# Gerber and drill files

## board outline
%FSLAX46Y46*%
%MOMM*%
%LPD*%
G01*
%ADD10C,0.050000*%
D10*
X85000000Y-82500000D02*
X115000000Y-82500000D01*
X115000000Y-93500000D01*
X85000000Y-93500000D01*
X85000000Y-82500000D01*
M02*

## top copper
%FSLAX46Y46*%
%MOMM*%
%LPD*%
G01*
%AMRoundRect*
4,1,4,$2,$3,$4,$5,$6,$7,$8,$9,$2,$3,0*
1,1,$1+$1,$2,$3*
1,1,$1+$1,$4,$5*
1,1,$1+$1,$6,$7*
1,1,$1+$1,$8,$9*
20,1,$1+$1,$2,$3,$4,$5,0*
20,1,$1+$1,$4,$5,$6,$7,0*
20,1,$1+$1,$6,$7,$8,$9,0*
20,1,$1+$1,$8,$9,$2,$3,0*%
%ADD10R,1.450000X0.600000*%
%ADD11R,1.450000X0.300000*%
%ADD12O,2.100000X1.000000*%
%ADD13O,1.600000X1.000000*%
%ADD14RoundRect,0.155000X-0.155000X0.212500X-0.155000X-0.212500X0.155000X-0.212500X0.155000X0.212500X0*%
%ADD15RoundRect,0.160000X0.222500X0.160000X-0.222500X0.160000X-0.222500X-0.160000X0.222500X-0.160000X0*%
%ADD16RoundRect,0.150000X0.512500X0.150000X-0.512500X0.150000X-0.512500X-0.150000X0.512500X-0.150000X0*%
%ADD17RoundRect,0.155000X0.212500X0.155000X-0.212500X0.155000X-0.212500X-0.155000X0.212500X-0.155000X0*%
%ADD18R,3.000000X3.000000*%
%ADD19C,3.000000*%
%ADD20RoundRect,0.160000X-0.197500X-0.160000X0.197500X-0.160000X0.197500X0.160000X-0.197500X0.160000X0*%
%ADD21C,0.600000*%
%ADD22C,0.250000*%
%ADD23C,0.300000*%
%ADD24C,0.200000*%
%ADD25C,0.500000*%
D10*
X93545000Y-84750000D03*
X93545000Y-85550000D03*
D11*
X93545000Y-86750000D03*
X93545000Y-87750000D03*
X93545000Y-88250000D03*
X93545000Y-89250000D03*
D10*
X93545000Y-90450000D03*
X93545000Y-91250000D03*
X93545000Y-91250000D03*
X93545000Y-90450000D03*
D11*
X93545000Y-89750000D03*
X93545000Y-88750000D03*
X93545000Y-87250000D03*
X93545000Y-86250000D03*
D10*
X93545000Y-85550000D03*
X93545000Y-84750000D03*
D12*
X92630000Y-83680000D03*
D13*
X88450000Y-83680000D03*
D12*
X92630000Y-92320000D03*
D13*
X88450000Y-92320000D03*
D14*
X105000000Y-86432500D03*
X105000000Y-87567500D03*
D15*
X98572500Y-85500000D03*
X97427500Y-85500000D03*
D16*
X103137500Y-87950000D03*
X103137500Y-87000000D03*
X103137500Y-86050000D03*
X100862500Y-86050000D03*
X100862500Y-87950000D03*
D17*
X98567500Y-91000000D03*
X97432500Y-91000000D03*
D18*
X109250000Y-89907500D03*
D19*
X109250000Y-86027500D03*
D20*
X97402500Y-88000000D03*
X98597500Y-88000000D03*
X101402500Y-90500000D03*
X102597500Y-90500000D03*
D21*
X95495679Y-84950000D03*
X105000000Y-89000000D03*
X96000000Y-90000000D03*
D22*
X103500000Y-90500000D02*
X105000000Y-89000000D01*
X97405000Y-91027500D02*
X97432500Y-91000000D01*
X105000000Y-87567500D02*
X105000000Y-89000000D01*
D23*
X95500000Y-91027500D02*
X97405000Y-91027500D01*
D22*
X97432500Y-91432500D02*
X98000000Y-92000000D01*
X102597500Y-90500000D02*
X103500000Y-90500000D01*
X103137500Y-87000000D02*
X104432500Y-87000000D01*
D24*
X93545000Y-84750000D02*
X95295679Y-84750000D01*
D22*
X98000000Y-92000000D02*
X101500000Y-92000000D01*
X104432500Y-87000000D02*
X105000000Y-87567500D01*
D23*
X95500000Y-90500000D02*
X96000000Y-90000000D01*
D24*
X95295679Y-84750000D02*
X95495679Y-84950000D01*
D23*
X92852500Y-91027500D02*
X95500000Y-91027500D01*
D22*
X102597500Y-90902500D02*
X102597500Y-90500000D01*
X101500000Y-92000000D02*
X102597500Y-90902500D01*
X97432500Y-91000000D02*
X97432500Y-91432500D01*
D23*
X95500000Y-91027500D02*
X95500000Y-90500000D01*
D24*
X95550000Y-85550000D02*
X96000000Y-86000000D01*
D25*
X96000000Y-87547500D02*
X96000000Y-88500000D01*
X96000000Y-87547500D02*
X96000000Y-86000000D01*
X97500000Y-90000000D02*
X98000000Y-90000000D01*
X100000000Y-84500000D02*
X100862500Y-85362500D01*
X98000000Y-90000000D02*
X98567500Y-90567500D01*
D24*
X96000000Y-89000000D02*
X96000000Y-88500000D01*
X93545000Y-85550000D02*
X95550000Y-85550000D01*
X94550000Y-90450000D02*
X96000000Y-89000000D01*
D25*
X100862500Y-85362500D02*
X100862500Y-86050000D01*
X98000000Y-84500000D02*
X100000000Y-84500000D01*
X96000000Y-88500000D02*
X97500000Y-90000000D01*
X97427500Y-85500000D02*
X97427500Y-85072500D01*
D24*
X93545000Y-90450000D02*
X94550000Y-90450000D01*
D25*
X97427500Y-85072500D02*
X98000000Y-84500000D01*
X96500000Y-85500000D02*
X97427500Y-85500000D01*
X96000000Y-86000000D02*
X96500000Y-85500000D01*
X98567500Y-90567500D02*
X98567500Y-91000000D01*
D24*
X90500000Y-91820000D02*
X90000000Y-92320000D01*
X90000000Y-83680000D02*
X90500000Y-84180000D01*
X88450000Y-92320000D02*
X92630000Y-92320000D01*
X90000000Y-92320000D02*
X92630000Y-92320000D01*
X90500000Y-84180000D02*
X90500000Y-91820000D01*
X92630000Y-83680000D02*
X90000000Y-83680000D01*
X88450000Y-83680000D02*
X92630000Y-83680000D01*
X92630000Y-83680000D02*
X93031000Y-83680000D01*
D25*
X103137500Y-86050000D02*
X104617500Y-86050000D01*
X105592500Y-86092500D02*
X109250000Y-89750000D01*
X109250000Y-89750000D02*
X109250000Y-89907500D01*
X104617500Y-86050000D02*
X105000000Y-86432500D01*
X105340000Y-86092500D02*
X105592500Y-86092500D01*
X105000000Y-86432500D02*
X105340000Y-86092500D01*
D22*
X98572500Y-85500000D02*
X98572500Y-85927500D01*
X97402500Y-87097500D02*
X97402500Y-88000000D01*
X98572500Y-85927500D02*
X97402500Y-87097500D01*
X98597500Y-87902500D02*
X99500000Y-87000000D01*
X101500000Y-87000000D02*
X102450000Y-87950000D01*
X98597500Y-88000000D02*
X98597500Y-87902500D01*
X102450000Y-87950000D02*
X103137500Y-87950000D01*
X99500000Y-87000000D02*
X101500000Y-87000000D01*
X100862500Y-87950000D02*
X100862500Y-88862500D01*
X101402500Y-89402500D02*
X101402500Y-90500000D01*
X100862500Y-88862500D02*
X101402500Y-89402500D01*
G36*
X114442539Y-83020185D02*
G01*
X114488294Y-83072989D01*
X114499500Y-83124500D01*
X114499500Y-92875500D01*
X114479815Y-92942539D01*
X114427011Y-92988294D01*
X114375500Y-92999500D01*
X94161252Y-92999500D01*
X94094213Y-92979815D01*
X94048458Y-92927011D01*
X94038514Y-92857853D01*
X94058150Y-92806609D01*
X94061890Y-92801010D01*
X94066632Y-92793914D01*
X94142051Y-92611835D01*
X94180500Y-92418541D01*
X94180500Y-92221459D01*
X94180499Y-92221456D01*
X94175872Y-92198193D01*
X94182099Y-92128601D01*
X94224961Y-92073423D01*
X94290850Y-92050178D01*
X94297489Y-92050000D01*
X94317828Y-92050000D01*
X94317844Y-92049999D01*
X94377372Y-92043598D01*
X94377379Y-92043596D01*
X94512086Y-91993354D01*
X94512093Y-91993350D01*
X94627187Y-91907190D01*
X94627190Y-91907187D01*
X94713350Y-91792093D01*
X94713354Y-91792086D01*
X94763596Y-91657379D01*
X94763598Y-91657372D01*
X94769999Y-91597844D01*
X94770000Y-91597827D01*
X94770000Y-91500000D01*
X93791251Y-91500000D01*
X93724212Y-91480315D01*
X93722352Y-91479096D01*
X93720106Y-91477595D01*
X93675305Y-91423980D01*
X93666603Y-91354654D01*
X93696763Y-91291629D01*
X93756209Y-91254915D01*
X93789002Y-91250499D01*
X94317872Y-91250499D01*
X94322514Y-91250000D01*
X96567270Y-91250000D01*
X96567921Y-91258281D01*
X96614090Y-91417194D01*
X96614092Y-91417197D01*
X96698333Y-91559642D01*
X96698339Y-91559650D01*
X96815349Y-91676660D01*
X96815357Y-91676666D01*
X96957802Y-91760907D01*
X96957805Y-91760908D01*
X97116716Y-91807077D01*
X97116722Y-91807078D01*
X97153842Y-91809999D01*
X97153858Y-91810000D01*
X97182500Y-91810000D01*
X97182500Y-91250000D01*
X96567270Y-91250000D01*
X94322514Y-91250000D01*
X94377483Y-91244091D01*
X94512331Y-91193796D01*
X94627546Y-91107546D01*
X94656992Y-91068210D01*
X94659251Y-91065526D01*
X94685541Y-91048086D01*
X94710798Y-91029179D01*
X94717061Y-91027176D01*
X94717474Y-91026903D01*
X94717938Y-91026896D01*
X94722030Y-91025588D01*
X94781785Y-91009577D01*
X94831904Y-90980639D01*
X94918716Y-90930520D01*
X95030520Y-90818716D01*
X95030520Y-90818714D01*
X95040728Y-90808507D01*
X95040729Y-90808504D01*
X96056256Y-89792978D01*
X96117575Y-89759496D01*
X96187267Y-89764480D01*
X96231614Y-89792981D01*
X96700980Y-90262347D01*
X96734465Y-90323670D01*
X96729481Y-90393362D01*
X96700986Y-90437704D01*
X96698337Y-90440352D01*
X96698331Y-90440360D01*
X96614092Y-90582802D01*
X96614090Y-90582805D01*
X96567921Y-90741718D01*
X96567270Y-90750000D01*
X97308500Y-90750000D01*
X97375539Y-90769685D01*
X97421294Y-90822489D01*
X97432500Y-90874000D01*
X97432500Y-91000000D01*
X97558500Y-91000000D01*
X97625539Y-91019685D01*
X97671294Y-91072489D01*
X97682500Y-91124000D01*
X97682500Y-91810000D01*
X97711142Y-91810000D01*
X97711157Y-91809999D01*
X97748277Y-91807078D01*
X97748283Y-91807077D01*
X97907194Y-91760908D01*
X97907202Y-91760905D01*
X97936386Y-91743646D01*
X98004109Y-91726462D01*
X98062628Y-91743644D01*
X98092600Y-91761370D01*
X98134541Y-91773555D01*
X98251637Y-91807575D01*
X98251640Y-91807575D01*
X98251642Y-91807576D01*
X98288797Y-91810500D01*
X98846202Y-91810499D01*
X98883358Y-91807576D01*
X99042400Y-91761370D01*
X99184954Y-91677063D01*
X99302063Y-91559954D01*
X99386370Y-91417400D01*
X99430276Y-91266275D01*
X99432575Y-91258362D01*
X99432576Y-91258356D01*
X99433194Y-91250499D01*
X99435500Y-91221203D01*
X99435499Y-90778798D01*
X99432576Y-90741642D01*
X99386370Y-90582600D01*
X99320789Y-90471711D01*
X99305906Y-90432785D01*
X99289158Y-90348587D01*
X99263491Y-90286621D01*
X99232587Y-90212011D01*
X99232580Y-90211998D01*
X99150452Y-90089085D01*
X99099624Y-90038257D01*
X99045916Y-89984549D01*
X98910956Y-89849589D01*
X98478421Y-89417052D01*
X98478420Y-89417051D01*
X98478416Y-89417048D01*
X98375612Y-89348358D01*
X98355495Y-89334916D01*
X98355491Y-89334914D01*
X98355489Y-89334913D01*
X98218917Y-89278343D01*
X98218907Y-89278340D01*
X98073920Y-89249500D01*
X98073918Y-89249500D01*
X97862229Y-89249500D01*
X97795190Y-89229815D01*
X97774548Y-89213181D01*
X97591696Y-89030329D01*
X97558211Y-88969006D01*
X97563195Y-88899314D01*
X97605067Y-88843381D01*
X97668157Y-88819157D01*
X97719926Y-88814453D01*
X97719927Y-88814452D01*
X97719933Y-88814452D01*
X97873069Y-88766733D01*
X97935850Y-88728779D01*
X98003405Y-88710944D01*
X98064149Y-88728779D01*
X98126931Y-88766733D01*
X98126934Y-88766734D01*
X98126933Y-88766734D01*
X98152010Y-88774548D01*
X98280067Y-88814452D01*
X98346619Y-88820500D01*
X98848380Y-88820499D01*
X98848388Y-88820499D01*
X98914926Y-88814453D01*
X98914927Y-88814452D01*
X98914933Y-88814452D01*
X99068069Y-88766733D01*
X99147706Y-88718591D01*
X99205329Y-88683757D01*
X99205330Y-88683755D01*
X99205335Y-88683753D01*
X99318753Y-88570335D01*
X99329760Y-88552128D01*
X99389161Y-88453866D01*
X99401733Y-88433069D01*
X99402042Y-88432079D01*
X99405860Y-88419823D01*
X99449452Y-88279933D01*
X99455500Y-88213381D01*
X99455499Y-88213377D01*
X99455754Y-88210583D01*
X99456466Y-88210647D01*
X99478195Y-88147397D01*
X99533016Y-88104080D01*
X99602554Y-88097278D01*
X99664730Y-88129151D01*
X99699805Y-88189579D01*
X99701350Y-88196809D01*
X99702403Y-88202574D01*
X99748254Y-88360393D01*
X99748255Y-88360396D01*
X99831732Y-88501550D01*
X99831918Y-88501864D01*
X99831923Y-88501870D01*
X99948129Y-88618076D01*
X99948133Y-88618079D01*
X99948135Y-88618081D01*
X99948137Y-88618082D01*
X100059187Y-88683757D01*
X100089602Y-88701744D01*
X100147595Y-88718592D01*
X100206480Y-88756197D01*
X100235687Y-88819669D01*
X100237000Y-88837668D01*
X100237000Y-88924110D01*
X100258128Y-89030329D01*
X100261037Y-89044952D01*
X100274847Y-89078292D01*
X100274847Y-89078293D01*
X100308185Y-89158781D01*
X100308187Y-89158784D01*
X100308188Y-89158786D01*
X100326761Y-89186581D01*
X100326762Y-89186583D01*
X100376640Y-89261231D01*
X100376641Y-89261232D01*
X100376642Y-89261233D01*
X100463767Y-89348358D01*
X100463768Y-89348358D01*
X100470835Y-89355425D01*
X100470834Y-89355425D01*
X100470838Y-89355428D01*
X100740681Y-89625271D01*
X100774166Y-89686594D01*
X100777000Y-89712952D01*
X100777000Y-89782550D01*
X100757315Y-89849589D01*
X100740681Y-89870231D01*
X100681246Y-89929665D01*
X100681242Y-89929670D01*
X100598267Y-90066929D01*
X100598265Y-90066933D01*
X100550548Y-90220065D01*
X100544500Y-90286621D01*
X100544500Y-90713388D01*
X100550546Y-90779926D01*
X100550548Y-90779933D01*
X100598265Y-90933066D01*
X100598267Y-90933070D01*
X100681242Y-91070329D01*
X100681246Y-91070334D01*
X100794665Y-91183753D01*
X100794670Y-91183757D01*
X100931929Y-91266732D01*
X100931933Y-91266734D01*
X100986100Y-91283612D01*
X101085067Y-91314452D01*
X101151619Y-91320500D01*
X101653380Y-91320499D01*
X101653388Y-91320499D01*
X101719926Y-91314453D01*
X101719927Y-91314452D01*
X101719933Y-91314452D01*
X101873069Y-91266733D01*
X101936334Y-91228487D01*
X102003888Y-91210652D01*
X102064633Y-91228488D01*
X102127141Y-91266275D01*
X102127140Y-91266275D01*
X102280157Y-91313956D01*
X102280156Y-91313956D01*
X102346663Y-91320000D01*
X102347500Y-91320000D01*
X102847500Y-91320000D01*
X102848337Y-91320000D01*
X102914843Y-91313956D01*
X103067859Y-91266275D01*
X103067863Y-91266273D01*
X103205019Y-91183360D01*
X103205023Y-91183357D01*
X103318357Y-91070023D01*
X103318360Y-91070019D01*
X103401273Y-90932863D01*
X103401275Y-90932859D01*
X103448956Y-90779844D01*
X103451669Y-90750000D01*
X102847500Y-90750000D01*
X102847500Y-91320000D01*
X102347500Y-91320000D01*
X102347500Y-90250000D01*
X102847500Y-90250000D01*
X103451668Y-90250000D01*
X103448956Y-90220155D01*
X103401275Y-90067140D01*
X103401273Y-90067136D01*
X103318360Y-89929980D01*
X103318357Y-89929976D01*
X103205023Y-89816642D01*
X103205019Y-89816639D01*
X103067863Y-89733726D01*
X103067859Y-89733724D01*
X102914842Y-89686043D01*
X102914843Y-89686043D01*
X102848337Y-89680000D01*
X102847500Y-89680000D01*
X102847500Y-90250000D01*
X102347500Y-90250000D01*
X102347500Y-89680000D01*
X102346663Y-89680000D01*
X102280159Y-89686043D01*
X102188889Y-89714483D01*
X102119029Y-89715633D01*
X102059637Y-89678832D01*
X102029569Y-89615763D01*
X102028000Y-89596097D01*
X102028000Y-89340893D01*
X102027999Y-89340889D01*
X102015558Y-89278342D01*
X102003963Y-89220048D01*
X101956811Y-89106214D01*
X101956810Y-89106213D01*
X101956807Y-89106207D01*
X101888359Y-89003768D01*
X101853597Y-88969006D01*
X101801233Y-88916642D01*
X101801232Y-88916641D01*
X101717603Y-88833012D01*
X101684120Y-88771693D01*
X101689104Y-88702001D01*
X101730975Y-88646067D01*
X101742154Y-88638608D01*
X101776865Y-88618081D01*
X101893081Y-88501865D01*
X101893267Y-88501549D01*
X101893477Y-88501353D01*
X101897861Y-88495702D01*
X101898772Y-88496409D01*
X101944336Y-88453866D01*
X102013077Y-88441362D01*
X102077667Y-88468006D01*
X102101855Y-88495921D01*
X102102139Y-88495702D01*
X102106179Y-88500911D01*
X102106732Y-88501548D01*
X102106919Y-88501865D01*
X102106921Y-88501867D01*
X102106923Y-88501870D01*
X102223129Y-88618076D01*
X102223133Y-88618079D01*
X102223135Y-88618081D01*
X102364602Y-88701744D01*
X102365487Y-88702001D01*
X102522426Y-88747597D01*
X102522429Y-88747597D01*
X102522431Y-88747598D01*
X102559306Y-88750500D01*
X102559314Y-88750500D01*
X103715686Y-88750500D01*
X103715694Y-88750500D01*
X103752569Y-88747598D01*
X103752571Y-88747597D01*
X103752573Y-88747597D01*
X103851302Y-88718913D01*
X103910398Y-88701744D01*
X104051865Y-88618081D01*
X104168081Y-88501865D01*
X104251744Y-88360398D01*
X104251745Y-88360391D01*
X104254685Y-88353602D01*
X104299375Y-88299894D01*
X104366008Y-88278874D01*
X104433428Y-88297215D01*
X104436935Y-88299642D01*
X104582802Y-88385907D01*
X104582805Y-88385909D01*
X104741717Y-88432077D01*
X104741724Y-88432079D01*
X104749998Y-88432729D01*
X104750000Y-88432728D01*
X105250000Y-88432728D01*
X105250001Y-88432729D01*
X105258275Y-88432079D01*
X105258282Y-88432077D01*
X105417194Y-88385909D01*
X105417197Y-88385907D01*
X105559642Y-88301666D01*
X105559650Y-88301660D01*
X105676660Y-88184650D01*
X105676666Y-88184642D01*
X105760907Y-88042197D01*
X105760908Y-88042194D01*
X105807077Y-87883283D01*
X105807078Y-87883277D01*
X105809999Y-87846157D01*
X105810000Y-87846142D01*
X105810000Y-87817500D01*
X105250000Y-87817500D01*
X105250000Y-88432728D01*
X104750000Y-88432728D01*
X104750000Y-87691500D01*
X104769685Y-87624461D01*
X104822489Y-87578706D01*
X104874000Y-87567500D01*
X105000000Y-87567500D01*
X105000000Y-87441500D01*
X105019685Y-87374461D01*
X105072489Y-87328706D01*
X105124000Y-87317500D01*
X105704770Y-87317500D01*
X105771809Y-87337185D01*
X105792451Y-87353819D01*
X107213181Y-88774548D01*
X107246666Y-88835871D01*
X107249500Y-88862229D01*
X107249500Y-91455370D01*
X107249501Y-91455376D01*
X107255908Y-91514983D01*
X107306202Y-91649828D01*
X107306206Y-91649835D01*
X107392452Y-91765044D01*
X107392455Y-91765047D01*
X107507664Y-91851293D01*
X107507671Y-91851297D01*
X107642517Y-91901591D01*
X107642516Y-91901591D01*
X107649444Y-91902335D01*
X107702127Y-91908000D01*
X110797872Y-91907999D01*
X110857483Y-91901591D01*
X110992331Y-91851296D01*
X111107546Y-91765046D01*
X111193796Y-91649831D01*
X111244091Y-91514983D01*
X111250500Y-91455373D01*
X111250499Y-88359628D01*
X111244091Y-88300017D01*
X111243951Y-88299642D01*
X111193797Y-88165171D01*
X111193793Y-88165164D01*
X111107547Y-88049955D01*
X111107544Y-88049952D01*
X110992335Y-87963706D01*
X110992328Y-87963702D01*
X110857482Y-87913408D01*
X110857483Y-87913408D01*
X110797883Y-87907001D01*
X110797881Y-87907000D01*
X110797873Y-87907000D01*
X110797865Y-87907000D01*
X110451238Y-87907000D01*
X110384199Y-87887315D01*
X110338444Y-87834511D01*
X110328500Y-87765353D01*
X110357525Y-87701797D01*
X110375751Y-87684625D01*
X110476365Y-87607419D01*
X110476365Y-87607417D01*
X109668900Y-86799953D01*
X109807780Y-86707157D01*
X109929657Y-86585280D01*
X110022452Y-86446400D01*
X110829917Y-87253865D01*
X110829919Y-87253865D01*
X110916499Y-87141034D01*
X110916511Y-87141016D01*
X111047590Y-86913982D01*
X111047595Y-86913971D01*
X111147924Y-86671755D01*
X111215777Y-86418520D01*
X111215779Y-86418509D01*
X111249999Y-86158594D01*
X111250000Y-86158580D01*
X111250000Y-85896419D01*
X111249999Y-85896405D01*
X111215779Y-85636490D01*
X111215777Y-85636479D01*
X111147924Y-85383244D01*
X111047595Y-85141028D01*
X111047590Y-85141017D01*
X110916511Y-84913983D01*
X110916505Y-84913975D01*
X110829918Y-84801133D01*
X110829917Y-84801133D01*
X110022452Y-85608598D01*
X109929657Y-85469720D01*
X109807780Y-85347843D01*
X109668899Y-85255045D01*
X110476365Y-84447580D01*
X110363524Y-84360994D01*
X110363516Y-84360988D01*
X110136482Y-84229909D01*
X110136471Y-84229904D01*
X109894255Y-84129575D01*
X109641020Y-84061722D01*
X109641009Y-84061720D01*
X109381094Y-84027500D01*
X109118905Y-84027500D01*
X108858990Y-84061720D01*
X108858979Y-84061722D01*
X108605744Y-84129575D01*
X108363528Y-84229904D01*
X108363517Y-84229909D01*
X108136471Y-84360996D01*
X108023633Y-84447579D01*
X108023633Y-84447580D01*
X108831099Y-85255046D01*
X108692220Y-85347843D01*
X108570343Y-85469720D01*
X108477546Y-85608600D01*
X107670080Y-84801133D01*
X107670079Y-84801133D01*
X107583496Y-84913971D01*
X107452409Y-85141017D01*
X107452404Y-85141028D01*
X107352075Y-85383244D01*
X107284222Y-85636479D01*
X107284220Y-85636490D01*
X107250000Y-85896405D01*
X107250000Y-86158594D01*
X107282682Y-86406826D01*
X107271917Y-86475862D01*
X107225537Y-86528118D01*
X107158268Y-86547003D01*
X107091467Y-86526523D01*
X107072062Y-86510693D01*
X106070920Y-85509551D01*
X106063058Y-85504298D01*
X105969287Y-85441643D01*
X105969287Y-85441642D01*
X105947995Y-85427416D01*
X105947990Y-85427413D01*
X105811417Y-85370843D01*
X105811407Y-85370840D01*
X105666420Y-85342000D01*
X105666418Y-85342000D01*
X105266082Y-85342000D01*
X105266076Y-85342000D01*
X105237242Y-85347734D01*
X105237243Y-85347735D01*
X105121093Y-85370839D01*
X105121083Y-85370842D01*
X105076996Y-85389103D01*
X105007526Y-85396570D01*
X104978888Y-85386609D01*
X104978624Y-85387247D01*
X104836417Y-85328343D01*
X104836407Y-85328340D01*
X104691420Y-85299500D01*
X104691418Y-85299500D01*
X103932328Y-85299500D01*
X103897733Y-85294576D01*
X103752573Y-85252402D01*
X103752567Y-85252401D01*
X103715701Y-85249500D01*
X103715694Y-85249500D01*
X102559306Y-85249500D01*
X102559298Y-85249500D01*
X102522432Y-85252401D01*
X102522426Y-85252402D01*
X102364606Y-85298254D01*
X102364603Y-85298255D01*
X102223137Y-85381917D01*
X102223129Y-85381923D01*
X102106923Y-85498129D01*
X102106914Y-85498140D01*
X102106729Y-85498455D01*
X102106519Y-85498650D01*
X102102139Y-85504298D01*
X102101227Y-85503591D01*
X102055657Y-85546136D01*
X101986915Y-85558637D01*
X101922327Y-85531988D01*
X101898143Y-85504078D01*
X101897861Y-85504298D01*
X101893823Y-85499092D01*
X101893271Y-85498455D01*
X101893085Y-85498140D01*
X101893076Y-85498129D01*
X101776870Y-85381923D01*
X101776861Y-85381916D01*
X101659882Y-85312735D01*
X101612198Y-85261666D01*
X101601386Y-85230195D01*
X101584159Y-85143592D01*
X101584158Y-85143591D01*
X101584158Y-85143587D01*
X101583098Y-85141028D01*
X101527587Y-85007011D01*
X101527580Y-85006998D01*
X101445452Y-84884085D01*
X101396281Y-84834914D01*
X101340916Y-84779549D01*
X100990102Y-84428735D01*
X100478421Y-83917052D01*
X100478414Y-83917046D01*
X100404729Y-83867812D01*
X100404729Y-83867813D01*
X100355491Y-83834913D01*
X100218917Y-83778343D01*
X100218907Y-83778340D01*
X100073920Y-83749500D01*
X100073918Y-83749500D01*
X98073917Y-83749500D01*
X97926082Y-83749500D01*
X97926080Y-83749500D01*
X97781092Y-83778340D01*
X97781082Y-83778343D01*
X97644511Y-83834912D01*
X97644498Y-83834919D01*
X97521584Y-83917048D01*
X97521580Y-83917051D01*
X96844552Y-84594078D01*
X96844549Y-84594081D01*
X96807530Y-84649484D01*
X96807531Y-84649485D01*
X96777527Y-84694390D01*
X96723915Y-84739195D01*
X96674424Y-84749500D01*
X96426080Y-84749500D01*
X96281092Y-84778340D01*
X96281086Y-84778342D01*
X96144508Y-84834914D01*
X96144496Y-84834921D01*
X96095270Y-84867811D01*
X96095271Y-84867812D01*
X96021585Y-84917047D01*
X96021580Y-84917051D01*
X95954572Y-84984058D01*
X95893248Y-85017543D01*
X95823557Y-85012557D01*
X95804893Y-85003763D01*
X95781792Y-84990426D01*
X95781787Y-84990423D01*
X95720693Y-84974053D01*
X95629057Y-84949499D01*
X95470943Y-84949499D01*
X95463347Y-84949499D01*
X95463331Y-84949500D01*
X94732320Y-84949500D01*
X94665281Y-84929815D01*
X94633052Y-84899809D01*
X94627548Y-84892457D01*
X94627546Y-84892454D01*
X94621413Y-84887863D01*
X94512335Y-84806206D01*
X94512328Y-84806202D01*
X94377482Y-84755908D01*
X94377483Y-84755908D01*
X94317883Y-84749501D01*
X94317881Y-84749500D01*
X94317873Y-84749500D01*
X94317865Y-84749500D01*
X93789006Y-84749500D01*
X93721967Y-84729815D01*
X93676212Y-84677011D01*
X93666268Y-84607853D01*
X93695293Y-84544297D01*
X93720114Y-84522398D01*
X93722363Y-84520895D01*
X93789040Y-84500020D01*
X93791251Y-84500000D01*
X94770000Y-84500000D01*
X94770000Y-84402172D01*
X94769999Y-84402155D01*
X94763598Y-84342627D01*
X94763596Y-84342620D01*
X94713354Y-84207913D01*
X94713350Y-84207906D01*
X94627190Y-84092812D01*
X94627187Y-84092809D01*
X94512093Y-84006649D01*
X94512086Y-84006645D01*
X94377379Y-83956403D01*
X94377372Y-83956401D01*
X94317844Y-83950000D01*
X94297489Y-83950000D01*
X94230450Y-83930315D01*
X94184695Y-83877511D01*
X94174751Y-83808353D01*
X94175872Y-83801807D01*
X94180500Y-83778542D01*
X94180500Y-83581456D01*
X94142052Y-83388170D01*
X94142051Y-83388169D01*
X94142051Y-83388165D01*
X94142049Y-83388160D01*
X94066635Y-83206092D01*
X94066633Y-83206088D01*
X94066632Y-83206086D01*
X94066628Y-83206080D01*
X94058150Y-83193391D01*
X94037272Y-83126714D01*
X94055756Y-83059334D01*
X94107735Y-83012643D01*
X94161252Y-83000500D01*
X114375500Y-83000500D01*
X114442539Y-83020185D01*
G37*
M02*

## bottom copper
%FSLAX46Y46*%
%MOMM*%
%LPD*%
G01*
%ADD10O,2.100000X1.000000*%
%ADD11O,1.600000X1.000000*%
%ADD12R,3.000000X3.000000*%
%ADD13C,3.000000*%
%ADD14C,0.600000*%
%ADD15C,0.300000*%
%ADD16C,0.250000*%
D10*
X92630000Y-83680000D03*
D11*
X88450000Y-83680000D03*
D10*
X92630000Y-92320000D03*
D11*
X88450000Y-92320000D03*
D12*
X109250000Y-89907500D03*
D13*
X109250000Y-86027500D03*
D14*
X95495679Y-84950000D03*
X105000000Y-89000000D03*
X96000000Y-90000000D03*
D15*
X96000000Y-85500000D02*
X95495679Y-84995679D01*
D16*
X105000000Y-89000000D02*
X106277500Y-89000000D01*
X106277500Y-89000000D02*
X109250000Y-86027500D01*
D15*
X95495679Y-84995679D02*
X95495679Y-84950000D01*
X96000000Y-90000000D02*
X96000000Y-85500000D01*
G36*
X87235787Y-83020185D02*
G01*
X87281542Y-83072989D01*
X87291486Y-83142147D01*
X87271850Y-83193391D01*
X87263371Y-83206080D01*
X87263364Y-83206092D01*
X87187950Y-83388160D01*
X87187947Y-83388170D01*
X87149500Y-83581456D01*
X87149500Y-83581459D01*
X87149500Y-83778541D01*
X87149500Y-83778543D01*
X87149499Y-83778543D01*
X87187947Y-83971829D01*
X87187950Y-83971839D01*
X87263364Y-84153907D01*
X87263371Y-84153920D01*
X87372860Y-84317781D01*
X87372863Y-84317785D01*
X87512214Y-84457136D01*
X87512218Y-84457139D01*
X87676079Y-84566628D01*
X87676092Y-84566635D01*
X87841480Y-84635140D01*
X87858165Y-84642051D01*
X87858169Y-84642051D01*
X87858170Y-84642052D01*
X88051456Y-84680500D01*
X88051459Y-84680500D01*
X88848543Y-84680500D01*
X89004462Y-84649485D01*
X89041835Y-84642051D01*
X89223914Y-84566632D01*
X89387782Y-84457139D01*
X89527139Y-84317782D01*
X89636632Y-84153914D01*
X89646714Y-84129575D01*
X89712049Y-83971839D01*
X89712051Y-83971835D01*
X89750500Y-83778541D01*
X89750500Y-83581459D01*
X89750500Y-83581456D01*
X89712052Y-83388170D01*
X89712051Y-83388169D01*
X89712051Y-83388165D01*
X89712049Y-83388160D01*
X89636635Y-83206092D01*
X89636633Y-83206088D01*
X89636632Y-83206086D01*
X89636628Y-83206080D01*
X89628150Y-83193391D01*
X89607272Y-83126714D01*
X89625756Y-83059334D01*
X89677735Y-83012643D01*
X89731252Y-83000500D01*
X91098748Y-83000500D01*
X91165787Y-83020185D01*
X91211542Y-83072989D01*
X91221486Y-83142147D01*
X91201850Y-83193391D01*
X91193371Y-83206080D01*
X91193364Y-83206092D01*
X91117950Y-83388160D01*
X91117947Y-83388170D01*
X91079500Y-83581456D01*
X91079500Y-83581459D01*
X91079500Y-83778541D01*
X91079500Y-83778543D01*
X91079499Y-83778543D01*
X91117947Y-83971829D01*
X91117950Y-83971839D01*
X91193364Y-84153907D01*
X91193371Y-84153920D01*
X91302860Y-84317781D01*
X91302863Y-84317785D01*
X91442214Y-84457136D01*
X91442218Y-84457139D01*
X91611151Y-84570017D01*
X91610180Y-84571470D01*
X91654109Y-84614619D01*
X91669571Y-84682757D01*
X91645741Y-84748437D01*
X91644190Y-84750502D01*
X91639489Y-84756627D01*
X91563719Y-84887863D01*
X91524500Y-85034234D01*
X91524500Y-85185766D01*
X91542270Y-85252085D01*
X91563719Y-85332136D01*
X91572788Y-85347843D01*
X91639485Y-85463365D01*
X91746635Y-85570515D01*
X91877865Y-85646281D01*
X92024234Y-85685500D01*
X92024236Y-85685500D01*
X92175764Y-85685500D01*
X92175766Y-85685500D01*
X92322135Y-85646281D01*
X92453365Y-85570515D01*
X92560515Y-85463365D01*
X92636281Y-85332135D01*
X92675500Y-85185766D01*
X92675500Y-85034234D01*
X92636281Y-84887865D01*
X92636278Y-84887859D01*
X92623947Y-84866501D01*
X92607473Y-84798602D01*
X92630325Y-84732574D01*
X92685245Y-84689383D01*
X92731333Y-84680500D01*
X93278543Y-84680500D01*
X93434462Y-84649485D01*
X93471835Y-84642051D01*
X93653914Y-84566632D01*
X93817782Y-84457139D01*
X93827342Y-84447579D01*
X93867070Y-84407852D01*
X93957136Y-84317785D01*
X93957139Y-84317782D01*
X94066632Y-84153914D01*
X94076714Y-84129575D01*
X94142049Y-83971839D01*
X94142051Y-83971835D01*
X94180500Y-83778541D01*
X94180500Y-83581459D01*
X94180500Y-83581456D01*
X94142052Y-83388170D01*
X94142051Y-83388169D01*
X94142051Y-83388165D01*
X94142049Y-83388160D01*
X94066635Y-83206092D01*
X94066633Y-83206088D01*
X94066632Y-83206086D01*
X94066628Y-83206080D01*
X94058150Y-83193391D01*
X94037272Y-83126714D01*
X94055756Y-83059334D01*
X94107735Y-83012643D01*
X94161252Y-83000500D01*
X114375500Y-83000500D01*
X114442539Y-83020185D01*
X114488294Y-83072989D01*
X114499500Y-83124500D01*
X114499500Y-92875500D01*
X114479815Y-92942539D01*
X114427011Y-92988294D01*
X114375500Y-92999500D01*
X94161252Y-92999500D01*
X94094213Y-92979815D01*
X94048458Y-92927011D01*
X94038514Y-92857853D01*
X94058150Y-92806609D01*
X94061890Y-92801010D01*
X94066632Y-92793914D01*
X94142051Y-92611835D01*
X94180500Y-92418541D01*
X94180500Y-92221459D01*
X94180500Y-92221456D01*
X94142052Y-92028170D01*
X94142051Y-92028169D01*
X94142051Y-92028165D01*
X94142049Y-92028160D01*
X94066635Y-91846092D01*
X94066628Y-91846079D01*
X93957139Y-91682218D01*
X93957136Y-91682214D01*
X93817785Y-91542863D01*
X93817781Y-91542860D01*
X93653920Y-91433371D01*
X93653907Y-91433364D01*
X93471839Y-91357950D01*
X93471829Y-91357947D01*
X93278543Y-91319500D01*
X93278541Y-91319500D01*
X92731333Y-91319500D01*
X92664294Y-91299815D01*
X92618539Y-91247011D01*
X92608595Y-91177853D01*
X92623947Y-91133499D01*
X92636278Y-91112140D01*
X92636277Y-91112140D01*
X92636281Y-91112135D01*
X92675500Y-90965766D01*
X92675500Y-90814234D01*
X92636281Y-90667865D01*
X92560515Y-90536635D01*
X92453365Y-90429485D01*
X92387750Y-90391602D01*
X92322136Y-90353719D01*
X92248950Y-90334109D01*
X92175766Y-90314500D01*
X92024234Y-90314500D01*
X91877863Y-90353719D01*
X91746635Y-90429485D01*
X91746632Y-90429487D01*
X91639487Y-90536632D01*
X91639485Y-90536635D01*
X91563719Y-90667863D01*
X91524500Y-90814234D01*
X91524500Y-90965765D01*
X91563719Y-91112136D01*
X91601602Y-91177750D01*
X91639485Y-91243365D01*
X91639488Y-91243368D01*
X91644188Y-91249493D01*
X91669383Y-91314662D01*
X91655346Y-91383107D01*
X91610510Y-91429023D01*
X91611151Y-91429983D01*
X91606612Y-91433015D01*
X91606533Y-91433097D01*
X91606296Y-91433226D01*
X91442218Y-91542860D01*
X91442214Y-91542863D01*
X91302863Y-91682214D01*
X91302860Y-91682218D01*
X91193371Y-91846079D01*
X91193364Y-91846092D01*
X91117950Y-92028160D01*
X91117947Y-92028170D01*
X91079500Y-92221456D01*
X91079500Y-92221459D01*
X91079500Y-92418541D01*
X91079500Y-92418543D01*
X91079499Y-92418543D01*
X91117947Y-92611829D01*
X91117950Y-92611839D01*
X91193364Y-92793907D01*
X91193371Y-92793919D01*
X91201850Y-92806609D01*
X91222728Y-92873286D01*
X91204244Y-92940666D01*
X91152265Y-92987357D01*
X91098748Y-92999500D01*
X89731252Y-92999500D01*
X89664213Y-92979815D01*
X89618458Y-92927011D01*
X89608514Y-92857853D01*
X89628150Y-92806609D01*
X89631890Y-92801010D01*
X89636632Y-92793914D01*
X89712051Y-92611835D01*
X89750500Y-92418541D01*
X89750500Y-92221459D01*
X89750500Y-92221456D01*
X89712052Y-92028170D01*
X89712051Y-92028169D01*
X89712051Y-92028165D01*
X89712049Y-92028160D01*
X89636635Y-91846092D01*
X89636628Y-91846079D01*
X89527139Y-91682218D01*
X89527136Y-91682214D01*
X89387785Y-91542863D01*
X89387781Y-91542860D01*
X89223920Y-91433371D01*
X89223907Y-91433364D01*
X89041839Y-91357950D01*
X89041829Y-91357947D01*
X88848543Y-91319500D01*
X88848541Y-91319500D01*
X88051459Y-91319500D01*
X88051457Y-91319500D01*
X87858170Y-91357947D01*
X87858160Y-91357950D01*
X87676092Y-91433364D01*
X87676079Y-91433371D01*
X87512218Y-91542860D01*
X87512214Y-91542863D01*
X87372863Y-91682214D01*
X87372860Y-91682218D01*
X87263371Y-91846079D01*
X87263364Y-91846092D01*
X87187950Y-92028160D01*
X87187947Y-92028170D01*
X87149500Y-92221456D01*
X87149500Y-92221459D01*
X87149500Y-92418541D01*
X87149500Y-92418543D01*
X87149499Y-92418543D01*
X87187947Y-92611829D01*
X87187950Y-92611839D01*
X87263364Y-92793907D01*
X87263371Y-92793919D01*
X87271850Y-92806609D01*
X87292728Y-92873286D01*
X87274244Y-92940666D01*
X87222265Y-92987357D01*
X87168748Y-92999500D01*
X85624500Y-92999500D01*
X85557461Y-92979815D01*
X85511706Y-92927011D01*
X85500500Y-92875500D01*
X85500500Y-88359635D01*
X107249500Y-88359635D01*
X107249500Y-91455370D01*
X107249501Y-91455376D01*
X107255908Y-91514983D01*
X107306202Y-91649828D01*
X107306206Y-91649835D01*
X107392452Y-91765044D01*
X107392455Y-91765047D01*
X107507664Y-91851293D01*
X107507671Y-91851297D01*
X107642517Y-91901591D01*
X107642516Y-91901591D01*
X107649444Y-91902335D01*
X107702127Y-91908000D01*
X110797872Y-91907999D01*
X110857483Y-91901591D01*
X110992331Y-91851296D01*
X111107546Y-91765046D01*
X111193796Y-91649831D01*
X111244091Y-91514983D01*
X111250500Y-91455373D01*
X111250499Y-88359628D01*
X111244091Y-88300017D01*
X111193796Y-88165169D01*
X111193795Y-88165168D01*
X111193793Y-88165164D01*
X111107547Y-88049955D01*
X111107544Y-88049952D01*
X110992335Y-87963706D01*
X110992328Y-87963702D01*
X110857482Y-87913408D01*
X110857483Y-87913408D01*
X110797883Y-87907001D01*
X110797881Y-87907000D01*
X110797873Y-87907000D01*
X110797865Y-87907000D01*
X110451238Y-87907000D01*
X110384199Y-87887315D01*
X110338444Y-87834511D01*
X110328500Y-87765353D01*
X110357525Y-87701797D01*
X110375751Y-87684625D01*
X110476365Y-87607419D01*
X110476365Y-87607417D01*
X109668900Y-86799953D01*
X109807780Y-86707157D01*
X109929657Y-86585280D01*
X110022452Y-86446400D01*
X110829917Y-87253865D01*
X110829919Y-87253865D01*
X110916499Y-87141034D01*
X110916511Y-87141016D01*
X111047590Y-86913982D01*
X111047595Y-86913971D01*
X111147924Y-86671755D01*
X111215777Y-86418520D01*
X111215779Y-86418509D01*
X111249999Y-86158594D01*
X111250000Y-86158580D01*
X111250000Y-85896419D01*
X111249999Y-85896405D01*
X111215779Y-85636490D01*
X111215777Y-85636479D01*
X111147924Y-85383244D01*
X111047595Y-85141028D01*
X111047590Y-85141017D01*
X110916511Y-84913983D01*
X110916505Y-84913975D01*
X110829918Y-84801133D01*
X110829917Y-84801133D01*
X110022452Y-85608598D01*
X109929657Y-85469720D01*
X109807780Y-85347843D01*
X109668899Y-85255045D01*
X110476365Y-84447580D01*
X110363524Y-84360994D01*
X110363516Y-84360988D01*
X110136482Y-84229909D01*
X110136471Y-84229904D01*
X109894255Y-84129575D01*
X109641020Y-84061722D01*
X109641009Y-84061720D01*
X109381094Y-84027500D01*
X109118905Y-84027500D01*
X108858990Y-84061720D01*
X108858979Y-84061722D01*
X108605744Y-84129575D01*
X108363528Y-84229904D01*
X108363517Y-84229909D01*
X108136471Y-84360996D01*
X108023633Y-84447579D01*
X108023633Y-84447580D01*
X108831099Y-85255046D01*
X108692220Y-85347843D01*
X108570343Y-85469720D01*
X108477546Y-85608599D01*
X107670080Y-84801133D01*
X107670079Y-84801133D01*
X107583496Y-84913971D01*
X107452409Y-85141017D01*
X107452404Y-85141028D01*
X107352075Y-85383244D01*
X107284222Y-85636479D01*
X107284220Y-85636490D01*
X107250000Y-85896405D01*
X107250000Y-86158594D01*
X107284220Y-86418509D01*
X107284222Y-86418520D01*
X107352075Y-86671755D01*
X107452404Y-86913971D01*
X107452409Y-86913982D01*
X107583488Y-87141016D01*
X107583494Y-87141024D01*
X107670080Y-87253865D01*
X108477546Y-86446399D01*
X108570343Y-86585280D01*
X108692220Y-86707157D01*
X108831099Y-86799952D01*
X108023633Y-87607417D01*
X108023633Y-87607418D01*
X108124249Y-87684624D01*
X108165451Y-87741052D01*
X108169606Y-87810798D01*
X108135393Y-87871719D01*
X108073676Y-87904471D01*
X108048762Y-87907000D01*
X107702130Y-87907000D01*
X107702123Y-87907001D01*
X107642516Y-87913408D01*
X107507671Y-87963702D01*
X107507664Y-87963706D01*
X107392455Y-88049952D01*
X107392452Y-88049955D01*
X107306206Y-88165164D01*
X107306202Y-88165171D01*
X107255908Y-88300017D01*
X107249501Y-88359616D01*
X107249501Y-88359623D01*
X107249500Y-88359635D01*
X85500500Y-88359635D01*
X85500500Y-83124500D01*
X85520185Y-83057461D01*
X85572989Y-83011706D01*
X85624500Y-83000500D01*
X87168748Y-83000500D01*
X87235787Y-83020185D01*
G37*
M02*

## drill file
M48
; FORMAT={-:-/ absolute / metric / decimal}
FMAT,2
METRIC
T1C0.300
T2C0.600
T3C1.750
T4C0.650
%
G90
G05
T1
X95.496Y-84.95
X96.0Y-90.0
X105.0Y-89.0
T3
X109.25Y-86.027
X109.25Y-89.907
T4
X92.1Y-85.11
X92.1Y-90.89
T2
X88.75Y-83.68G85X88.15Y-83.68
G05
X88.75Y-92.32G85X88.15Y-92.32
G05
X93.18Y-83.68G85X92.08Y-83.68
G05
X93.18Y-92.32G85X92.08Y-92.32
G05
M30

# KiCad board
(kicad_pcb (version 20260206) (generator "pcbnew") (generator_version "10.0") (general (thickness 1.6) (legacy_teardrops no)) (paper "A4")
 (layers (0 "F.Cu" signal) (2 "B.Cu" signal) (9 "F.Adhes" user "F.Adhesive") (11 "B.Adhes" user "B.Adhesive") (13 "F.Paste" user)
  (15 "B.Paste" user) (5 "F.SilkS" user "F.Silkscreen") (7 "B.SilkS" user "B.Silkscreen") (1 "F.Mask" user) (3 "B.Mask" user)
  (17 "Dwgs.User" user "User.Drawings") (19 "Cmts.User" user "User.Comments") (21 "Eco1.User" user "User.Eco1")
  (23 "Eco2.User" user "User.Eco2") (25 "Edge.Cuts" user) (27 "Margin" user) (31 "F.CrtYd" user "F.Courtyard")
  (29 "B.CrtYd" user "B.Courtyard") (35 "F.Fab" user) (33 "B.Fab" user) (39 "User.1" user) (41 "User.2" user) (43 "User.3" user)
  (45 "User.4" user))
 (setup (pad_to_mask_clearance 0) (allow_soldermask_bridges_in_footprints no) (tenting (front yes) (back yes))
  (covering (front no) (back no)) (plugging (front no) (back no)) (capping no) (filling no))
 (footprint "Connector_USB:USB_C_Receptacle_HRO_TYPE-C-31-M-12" (layer "F.Cu") (at 89.5 88 -90)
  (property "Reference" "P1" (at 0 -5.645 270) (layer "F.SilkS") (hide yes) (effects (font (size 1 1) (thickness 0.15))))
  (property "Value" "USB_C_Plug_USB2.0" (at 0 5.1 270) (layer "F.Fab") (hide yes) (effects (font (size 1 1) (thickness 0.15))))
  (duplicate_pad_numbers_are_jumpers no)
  (pad "" np_thru_hole circle (at -2.89 -2.6 270) (size 0.65 0.65) (drill 0.65) (layers "*.Cu" "*.Mask"))
  (pad "" np_thru_hole circle (at 2.89 -2.6 270) (size 0.65 0.65) (drill 0.65) (layers "*.Cu" "*.Mask"))
  (pad "A1" smd rect (at -3.25 -4.045 270) (size 0.6 1.45) (layers "F.Cu" "F.Mask" "F.Paste") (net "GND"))
  (pad "A4" smd rect (at -2.45 -4.045 270) (size 0.6 1.45) (layers "F.Cu" "F.Mask" "F.Paste") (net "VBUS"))
  (pad "A5" smd rect (at -1.25 -4.045 270) (size 0.3 1.45) (layers "F.Cu" "F.Mask" "F.Paste") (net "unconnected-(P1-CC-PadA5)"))
  (pad "A6" smd rect (at -0.25 -4.045 270) (size 0.3 1.45) (layers "F.Cu" "F.Mask" "F.Paste") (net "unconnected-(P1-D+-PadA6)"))
  (pad "A7" smd rect (at 0.25 -4.045 270) (size 0.3 1.45) (layers "F.Cu" "F.Mask" "F.Paste") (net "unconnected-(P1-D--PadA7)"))
  (pad "A8" smd rect (at 1.25 -4.045 270) (size 0.3 1.45) (layers "F.Cu" "F.Mask" "F.Paste"))
  (pad "A9" smd rect (at 2.45 -4.045 270) (size 0.6 1.45) (layers "F.Cu" "F.Mask" "F.Paste") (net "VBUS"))
  (pad "A12" smd rect (at 3.25 -4.045 270) (size 0.6 1.45) (layers "F.Cu" "F.Mask" "F.Paste") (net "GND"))
  (pad "B1" smd rect (at 3.25 -4.045 270) (size 0.6 1.45) (layers "F.Cu" "F.Mask" "F.Paste") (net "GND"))
  (pad "B4" smd rect (at 2.45 -4.045 270) (size 0.6 1.45) (layers "F.Cu" "F.Mask" "F.Paste") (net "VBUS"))
  (pad "B5" smd rect (at 1.75 -4.045 270) (size 0.3 1.45) (layers "F.Cu" "F.Mask" "F.Paste") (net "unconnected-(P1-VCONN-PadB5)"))
  (pad "B6" smd rect (at 0.75 -4.045 270) (size 0.3 1.45) (layers "F.Cu" "F.Mask" "F.Paste"))
  (pad "B7" smd rect (at -0.75 -4.045 270) (size 0.3 1.45) (layers "F.Cu" "F.Mask" "F.Paste"))
  (pad "B8" smd rect (at -1.75 -4.045 270) (size 0.3 1.45) (layers "F.Cu" "F.Mask" "F.Paste"))
  (pad "B9" smd rect (at -2.45 -4.045 270) (size 0.6 1.45) (layers "F.Cu" "F.Mask" "F.Paste") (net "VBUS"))
  (pad "B12" smd rect (at -3.25 -4.045 270) (size 0.6 1.45) (layers "F.Cu" "F.Mask" "F.Paste") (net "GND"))
  (pad "S1" thru_hole oval (at -4.32 -3.13 270) (size 1 2.1) (drill oval 0.6 1.7) (layers "*.Cu" "*.Mask") (remove_unused_layers no)
   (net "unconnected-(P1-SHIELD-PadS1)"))
  (pad "S1" thru_hole oval (at -4.32 1.05 270) (size 1 1.6) (drill oval 0.6 1.2) (layers "*.Cu" "*.Mask") (remove_unused_layers no)
   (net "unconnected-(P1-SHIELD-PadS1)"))
  (pad "S1" thru_hole oval (at 4.32 -3.13 270) (size 1 2.1) (drill oval 0.6 1.7) (layers "*.Cu" "*.Mask") (remove_unused_layers no)
   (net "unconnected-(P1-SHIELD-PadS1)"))
  (pad "S1" thru_hole oval (at 4.32 1.05 270) (size 1 1.6) (drill oval 0.6 1.2) (layers "*.Cu" "*.Mask") (remove_unused_layers no)
   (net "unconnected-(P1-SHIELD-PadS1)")))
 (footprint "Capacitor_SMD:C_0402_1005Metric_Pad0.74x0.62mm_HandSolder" (layer "F.Cu") (at 105 87 -90)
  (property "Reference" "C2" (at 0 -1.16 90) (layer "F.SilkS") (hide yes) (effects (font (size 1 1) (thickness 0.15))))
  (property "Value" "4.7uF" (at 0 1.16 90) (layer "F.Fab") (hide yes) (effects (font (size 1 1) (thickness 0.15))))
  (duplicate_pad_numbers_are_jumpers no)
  (pad "1" smd roundrect (at -0.5675 0 270) (size 0.735 0.62) (layers "F.Cu" "F.Mask" "F.Paste") (roundrect_rratio 0.25) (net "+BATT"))
  (pad "2" smd roundrect (at 0.5675 0 270) (size 0.735 0.62) (layers "F.Cu" "F.Mask" "F.Paste") (roundrect_rratio 0.25) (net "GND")))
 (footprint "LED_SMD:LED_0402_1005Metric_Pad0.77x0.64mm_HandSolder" (layer "F.Cu") (at 98 85.5 180)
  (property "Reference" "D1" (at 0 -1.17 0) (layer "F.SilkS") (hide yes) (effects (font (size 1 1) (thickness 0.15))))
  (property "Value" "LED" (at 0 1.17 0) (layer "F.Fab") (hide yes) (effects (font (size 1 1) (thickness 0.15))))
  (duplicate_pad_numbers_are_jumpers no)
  (pad "1" smd roundrect (at -0.5725 0 180) (size 0.765 0.64) (layers "F.Cu" "F.Mask" "F.Paste") (roundrect_rratio 0.25) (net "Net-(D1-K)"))
  (pad "2" smd roundrect (at 0.5725 0 180) (size 0.765 0.64) (layers "F.Cu" "F.Mask" "F.Paste") (roundrect_rratio 0.25) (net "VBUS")))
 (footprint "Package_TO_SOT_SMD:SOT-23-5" (layer "F.Cu") (at 102 87 180)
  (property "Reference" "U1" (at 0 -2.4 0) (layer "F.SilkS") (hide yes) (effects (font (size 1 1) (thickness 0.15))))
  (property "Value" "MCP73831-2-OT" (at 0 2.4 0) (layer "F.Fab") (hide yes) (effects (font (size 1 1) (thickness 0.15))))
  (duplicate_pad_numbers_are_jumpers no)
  (pad "1" smd roundrect (at -1.1375 -0.95 180) (size 1.325 0.6) (layers "F.Cu" "F.Mask" "F.Paste") (roundrect_rratio 0.25)
   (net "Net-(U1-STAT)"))
  (pad "2" smd roundrect (at -1.1375 0 180) (size 1.325 0.6) (layers "F.Cu" "F.Mask" "F.Paste") (roundrect_rratio 0.25) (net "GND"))
  (pad "3" smd roundrect (at -1.1375 0.95 180) (size 1.325 0.6) (layers "F.Cu" "F.Mask" "F.Paste") (roundrect_rratio 0.25) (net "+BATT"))
  (pad "4" smd roundrect (at 1.1375 0.95 180) (size 1.325 0.6) (layers "F.Cu" "F.Mask" "F.Paste") (roundrect_rratio 0.25) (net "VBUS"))
  (pad "5" smd roundrect (at 1.1375 -0.95 180) (size 1.325 0.6) (layers "F.Cu" "F.Mask" "F.Paste") (roundrect_rratio 0.25)
   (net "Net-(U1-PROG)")))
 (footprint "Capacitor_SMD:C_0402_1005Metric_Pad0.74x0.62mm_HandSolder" (layer "F.Cu") (at 98 91 180)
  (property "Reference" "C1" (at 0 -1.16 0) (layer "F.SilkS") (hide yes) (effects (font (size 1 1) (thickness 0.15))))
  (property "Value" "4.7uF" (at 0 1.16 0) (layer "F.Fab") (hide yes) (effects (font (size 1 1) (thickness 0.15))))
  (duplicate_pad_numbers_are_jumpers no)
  (pad "1" smd roundrect (at -0.5675 0 180) (size 0.735 0.62) (layers "F.Cu" "F.Mask" "F.Paste") (roundrect_rratio 0.25) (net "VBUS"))
  (pad "2" smd roundrect (at 0.5675 0 180) (size 0.735 0.62) (layers "F.Cu" "F.Mask" "F.Paste") (roundrect_rratio 0.25) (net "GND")))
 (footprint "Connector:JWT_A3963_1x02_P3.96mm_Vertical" (layer "F.Cu") (at 109.25 89.9075 90)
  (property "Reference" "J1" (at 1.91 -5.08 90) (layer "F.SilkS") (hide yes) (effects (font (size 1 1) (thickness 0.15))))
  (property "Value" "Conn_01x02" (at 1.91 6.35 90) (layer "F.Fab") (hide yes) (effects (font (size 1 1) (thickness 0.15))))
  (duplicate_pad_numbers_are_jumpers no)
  (pad "1" thru_hole rect (at 0 0 90) (size 3 3) (drill 1.75) (layers "*.Cu" "*.Mask") (remove_unused_layers no) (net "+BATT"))
  (pad "2" thru_hole circle (at 3.88 0 90) (size 3 3) (drill 1.75) (layers "*.Cu" "*.Mask") (remove_unused_layers no) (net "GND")))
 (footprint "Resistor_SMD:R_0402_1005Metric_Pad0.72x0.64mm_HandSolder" (layer "F.Cu") (at 98 88)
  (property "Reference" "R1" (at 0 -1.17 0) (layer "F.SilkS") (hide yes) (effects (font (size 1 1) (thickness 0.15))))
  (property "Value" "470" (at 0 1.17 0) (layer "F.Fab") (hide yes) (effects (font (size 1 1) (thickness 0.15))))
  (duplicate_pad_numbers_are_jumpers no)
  (pad "1" smd roundrect (at -0.5975 0) (size 0.715 0.64) (layers "F.Cu" "F.Mask" "F.Paste") (roundrect_rratio 0.25) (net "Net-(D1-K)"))
  (pad "2" smd roundrect (at 0.5975 0) (size 0.715 0.64) (layers "F.Cu" "F.Mask" "F.Paste") (roundrect_rratio 0.25) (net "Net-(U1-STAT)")))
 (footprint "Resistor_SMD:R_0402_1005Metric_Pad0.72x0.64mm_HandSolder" (layer "F.Cu") (at 102 90.5)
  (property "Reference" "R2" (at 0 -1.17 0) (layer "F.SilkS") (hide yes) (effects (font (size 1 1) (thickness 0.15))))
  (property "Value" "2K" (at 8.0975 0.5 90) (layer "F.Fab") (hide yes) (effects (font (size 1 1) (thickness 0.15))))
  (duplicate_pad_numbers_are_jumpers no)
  (pad "1" smd roundrect (at -0.5975 0) (size 0.715 0.64) (layers "F.Cu" "F.Mask" "F.Paste") (roundrect_rratio 0.25) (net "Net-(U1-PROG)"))
  (pad "2" smd roundrect (at 0.5975 0) (size 0.715 0.64) (layers "F.Cu" "F.Mask" "F.Paste") (roundrect_rratio 0.25) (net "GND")))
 (gr_rect (start 85 82.5) (end 115 93.5) (stroke (width 0.05) (type default)) (fill no) (layer "Edge.Cuts"))
 (segment (start 103.5 90.5) (end 105 89) (width 0.25) (layer "F.Cu") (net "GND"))
 (segment (start 97.405 91.0275) (end 97.4325 91) (width 0.25) (layer "F.Cu") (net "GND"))
 (segment (start 105 87.5675) (end 105 89) (width 0.25) (layer "F.Cu") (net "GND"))
 (segment (start 95.5 91.0275) (end 97.405 91.0275) (width 0.3) (layer "F.Cu") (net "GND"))
 (segment (start 97.4325 91.4325) (end 98 92) (width 0.25) (layer "F.Cu") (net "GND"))
 (segment (start 102.5975 90.5) (end 103.5 90.5) (width 0.25) (layer "F.Cu") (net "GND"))
 (segment (start 103.1375 87) (end 104.4325 87) (width 0.25) (layer "F.Cu") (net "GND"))
 (segment (start 93.545 84.75) (end 95.295679 84.75) (width 0.2) (layer "F.Cu") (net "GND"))
 (segment (start 98 92) (end 101.5 92) (width 0.25) (layer "F.Cu") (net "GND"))
 (segment (start 104.4325 87) (end 105 87.5675) (width 0.25) (layer "F.Cu") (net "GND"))
 (segment (start 95.5 90.5) (end 96 90) (width 0.3) (layer "F.Cu") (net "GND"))
 (segment (start 95.295679 84.75) (end 95.495679 84.95) (width 0.2) (layer "F.Cu") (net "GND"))
 (segment (start 92.8525 91.0275) (end 95.5 91.0275) (width 0.3) (layer "F.Cu") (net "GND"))
 (segment (start 102.5975 90.9025) (end 102.5975 90.5) (width 0.25) (layer "F.Cu") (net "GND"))
 (segment (start 101.5 92) (end 102.5975 90.9025) (width 0.25) (layer "F.Cu") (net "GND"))
 (segment (start 97.4325 91) (end 97.4325 91.4325) (width 0.25) (layer "F.Cu") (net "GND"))
 (segment (start 95.5 91.0275) (end 95.5 90.5) (width 0.3) (layer "F.Cu") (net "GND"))
 (via (at 95.495679 84.95) (size 0.6) (drill 0.3) (layers "F.Cu" "B.Cu") (capping no) (covering (front no) (back no))
  (plugging (front no) (back no)) (filling no) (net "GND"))
 (via (at 105 89) (size 0.6) (drill 0.3) (layers "F.Cu" "B.Cu") (capping no) (covering (front no) (back no)) (plugging (front no) (back no))
  (filling no) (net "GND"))
 (via (at 96 90) (size 0.6) (drill 0.3) (layers "F.Cu" "B.Cu") (capping no) (covering (front no) (back no)) (plugging (front no) (back no))
  (filling no) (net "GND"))
 (segment (start 96 85.5) (end 95.495679 84.995679) (width 0.3) (layer "B.Cu") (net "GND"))
 (segment (start 105 89) (end 106.2775 89) (width 0.25) (layer "B.Cu") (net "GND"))
 (segment (start 106.2775 89) (end 109.25 86.0275) (width 0.25) (layer "B.Cu") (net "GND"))
 (segment (start 95.495679 84.995679) (end 95.495679 84.95) (width 0.3) (layer "B.Cu") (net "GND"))
 (segment (start 96 90) (end 96 85.5) (width 0.3) (layer "B.Cu") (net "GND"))
 (segment (start 95.55 85.55) (end 96 86) (width 0.2) (layer "F.Cu") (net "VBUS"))
 (segment (start 96 87.5475) (end 96 88.5) (width 0.5) (layer "F.Cu") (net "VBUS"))
 (segment (start 96 87.5475) (end 96 86) (width 0.5) (layer "F.Cu") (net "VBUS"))
 (segment (start 97.5 90) (end 98 90) (width 0.5) (layer "F.Cu") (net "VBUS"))
 (segment (start 100 84.5) (end 100.8625 85.3625) (width 0.5) (layer "F.Cu") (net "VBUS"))
 (segment (start 98 90) (end 98.5675 90.5675) (width 0.5) (layer "F.Cu") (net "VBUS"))
 (segment (start 96 89) (end 96 88.5) (width 0.2) (layer "F.Cu") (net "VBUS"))
 (segment (start 93.545 85.55) (end 95.55 85.55) (width 0.2) (layer "F.Cu") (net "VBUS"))
 (segment (start 94.55 90.45) (end 96 89) (width 0.2) (layer "F.Cu") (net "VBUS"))
 (segment (start 100.8625 85.3625) (end 100.8625 86.05) (width 0.5) (layer "F.Cu") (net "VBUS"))
 (segment (start 98 84.5) (end 100 84.5) (width 0.5) (layer "F.Cu") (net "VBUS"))
 (segment (start 96 88.5) (end 97.5 90) (width 0.5) (layer "F.Cu") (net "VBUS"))
 (segment (start 97.4275 85.5) (end 97.4275 85.0725) (width 0.5) (layer "F.Cu") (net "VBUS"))
 (segment (start 93.545 90.45) (end 94.55 90.45) (width 0.2) (layer "F.Cu") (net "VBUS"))
 (segment (start 97.4275 85.0725) (end 98 84.5) (width 0.5) (layer "F.Cu") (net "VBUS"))
 (segment (start 96.5 85.5) (end 97.4275 85.5) (width 0.5) (layer "F.Cu") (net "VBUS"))
 (segment (start 96 86) (end 96.5 85.5) (width 0.5) (layer "F.Cu") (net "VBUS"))
 (segment (start 98.5675 90.5675) (end 98.5675 91) (width 0.5) (layer "F.Cu") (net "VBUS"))
 (segment (start 90.5 91.82) (end 90 92.32) (width 0.2) (layer "F.Cu") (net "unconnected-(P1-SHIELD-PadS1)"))
 (segment (start 90 83.68) (end 90.5 84.18) (width 0.2) (layer "F.Cu") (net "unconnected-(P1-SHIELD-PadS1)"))
 (segment (start 88.45 92.32) (end 92.63 92.32) (width 0.2) (layer "F.Cu") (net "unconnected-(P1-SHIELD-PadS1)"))
 (segment (start 90 92.32) (end 92.63 92.32) (width 0.2) (layer "F.Cu") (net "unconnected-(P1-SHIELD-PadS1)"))
 (segment (start 90.5 84.18) (end 90.5 91.82) (width 0.2) (layer "F.Cu") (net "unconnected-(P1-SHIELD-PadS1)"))
 (segment (start 92.63 83.68) (end 90 83.68) (width 0.2) (layer "F.Cu") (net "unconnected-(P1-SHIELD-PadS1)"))
 (segment (start 88.45 83.68) (end 92.63 83.68) (width 0.2) (layer "F.Cu") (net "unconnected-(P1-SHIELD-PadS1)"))
 (segment (start 92.63 83.68) (end 93.031 83.68) (width 0.2) (layer "F.Cu") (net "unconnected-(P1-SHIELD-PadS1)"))
 (segment (start 103.1375 86.05) (end 104.6175 86.05) (width 0.5) (layer "F.Cu") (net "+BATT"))
 (segment (start 105.5925 86.0925) (end 109.25 89.75) (width 0.5) (layer "F.Cu") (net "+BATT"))
 (segment (start 109.25 89.75) (end 109.25 89.9075) (width 0.5) (layer "F.Cu") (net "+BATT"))
 (segment (start 104.6175 86.05) (end 105 86.4325) (width 0.5) (layer "F.Cu") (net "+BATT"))
 (segment (start 105.34 86.0925) (end 105.5925 86.0925) (width 0.5) (layer "F.Cu") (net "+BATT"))
 (segment (start 105 86.4325) (end 105.34 86.0925) (width 0.5) (layer "F.Cu") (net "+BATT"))
 (segment (start 98.5725 85.5) (end 98.5725 85.9275) (width 0.25) (layer "F.Cu") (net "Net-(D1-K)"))
 (segment (start 97.4025 87.0975) (end 97.4025 88) (width 0.25) (layer "F.Cu") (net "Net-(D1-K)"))
 (segment (start 98.5725 85.9275) (end 97.4025 87.0975) (width 0.25) (layer "F.Cu") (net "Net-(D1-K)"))
 (segment (start 98.5975 87.9025) (end 99.5 87) (width 0.25) (layer "F.Cu") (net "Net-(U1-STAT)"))
 (segment (start 101.5 87) (end 102.45 87.95) (width 0.25) (layer "F.Cu") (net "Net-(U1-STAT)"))
 (segment (start 98.5975 88) (end 98.5975 87.9025) (width 0.25) (layer "F.Cu") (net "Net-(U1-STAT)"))
 (segment (start 102.45 87.95) (end 103.1375 87.95) (width 0.25) (layer "F.Cu") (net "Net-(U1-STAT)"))
 (segment (start 99.5 87) (end 101.5 87) (width 0.25) (layer "F.Cu") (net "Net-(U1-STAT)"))
 (segment (start 100.8625 87.95) (end 100.8625 88.8625) (width 0.25) (layer "F.Cu") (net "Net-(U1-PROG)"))
 (segment (start 101.4025 89.4025) (end 101.4025 90.5) (width 0.25) (layer "F.Cu") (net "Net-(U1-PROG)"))
 (segment (start 100.8625 88.8625) (end 101.4025 89.4025) (width 0.25) (layer "F.Cu") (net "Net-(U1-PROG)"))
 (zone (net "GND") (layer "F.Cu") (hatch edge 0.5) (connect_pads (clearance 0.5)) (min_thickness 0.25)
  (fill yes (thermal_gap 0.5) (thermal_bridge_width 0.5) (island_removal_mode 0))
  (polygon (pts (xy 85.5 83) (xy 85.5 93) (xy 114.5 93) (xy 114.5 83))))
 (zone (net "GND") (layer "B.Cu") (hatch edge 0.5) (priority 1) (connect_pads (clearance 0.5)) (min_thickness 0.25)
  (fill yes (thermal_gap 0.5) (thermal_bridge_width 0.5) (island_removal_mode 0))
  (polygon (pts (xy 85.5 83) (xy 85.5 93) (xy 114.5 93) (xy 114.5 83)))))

